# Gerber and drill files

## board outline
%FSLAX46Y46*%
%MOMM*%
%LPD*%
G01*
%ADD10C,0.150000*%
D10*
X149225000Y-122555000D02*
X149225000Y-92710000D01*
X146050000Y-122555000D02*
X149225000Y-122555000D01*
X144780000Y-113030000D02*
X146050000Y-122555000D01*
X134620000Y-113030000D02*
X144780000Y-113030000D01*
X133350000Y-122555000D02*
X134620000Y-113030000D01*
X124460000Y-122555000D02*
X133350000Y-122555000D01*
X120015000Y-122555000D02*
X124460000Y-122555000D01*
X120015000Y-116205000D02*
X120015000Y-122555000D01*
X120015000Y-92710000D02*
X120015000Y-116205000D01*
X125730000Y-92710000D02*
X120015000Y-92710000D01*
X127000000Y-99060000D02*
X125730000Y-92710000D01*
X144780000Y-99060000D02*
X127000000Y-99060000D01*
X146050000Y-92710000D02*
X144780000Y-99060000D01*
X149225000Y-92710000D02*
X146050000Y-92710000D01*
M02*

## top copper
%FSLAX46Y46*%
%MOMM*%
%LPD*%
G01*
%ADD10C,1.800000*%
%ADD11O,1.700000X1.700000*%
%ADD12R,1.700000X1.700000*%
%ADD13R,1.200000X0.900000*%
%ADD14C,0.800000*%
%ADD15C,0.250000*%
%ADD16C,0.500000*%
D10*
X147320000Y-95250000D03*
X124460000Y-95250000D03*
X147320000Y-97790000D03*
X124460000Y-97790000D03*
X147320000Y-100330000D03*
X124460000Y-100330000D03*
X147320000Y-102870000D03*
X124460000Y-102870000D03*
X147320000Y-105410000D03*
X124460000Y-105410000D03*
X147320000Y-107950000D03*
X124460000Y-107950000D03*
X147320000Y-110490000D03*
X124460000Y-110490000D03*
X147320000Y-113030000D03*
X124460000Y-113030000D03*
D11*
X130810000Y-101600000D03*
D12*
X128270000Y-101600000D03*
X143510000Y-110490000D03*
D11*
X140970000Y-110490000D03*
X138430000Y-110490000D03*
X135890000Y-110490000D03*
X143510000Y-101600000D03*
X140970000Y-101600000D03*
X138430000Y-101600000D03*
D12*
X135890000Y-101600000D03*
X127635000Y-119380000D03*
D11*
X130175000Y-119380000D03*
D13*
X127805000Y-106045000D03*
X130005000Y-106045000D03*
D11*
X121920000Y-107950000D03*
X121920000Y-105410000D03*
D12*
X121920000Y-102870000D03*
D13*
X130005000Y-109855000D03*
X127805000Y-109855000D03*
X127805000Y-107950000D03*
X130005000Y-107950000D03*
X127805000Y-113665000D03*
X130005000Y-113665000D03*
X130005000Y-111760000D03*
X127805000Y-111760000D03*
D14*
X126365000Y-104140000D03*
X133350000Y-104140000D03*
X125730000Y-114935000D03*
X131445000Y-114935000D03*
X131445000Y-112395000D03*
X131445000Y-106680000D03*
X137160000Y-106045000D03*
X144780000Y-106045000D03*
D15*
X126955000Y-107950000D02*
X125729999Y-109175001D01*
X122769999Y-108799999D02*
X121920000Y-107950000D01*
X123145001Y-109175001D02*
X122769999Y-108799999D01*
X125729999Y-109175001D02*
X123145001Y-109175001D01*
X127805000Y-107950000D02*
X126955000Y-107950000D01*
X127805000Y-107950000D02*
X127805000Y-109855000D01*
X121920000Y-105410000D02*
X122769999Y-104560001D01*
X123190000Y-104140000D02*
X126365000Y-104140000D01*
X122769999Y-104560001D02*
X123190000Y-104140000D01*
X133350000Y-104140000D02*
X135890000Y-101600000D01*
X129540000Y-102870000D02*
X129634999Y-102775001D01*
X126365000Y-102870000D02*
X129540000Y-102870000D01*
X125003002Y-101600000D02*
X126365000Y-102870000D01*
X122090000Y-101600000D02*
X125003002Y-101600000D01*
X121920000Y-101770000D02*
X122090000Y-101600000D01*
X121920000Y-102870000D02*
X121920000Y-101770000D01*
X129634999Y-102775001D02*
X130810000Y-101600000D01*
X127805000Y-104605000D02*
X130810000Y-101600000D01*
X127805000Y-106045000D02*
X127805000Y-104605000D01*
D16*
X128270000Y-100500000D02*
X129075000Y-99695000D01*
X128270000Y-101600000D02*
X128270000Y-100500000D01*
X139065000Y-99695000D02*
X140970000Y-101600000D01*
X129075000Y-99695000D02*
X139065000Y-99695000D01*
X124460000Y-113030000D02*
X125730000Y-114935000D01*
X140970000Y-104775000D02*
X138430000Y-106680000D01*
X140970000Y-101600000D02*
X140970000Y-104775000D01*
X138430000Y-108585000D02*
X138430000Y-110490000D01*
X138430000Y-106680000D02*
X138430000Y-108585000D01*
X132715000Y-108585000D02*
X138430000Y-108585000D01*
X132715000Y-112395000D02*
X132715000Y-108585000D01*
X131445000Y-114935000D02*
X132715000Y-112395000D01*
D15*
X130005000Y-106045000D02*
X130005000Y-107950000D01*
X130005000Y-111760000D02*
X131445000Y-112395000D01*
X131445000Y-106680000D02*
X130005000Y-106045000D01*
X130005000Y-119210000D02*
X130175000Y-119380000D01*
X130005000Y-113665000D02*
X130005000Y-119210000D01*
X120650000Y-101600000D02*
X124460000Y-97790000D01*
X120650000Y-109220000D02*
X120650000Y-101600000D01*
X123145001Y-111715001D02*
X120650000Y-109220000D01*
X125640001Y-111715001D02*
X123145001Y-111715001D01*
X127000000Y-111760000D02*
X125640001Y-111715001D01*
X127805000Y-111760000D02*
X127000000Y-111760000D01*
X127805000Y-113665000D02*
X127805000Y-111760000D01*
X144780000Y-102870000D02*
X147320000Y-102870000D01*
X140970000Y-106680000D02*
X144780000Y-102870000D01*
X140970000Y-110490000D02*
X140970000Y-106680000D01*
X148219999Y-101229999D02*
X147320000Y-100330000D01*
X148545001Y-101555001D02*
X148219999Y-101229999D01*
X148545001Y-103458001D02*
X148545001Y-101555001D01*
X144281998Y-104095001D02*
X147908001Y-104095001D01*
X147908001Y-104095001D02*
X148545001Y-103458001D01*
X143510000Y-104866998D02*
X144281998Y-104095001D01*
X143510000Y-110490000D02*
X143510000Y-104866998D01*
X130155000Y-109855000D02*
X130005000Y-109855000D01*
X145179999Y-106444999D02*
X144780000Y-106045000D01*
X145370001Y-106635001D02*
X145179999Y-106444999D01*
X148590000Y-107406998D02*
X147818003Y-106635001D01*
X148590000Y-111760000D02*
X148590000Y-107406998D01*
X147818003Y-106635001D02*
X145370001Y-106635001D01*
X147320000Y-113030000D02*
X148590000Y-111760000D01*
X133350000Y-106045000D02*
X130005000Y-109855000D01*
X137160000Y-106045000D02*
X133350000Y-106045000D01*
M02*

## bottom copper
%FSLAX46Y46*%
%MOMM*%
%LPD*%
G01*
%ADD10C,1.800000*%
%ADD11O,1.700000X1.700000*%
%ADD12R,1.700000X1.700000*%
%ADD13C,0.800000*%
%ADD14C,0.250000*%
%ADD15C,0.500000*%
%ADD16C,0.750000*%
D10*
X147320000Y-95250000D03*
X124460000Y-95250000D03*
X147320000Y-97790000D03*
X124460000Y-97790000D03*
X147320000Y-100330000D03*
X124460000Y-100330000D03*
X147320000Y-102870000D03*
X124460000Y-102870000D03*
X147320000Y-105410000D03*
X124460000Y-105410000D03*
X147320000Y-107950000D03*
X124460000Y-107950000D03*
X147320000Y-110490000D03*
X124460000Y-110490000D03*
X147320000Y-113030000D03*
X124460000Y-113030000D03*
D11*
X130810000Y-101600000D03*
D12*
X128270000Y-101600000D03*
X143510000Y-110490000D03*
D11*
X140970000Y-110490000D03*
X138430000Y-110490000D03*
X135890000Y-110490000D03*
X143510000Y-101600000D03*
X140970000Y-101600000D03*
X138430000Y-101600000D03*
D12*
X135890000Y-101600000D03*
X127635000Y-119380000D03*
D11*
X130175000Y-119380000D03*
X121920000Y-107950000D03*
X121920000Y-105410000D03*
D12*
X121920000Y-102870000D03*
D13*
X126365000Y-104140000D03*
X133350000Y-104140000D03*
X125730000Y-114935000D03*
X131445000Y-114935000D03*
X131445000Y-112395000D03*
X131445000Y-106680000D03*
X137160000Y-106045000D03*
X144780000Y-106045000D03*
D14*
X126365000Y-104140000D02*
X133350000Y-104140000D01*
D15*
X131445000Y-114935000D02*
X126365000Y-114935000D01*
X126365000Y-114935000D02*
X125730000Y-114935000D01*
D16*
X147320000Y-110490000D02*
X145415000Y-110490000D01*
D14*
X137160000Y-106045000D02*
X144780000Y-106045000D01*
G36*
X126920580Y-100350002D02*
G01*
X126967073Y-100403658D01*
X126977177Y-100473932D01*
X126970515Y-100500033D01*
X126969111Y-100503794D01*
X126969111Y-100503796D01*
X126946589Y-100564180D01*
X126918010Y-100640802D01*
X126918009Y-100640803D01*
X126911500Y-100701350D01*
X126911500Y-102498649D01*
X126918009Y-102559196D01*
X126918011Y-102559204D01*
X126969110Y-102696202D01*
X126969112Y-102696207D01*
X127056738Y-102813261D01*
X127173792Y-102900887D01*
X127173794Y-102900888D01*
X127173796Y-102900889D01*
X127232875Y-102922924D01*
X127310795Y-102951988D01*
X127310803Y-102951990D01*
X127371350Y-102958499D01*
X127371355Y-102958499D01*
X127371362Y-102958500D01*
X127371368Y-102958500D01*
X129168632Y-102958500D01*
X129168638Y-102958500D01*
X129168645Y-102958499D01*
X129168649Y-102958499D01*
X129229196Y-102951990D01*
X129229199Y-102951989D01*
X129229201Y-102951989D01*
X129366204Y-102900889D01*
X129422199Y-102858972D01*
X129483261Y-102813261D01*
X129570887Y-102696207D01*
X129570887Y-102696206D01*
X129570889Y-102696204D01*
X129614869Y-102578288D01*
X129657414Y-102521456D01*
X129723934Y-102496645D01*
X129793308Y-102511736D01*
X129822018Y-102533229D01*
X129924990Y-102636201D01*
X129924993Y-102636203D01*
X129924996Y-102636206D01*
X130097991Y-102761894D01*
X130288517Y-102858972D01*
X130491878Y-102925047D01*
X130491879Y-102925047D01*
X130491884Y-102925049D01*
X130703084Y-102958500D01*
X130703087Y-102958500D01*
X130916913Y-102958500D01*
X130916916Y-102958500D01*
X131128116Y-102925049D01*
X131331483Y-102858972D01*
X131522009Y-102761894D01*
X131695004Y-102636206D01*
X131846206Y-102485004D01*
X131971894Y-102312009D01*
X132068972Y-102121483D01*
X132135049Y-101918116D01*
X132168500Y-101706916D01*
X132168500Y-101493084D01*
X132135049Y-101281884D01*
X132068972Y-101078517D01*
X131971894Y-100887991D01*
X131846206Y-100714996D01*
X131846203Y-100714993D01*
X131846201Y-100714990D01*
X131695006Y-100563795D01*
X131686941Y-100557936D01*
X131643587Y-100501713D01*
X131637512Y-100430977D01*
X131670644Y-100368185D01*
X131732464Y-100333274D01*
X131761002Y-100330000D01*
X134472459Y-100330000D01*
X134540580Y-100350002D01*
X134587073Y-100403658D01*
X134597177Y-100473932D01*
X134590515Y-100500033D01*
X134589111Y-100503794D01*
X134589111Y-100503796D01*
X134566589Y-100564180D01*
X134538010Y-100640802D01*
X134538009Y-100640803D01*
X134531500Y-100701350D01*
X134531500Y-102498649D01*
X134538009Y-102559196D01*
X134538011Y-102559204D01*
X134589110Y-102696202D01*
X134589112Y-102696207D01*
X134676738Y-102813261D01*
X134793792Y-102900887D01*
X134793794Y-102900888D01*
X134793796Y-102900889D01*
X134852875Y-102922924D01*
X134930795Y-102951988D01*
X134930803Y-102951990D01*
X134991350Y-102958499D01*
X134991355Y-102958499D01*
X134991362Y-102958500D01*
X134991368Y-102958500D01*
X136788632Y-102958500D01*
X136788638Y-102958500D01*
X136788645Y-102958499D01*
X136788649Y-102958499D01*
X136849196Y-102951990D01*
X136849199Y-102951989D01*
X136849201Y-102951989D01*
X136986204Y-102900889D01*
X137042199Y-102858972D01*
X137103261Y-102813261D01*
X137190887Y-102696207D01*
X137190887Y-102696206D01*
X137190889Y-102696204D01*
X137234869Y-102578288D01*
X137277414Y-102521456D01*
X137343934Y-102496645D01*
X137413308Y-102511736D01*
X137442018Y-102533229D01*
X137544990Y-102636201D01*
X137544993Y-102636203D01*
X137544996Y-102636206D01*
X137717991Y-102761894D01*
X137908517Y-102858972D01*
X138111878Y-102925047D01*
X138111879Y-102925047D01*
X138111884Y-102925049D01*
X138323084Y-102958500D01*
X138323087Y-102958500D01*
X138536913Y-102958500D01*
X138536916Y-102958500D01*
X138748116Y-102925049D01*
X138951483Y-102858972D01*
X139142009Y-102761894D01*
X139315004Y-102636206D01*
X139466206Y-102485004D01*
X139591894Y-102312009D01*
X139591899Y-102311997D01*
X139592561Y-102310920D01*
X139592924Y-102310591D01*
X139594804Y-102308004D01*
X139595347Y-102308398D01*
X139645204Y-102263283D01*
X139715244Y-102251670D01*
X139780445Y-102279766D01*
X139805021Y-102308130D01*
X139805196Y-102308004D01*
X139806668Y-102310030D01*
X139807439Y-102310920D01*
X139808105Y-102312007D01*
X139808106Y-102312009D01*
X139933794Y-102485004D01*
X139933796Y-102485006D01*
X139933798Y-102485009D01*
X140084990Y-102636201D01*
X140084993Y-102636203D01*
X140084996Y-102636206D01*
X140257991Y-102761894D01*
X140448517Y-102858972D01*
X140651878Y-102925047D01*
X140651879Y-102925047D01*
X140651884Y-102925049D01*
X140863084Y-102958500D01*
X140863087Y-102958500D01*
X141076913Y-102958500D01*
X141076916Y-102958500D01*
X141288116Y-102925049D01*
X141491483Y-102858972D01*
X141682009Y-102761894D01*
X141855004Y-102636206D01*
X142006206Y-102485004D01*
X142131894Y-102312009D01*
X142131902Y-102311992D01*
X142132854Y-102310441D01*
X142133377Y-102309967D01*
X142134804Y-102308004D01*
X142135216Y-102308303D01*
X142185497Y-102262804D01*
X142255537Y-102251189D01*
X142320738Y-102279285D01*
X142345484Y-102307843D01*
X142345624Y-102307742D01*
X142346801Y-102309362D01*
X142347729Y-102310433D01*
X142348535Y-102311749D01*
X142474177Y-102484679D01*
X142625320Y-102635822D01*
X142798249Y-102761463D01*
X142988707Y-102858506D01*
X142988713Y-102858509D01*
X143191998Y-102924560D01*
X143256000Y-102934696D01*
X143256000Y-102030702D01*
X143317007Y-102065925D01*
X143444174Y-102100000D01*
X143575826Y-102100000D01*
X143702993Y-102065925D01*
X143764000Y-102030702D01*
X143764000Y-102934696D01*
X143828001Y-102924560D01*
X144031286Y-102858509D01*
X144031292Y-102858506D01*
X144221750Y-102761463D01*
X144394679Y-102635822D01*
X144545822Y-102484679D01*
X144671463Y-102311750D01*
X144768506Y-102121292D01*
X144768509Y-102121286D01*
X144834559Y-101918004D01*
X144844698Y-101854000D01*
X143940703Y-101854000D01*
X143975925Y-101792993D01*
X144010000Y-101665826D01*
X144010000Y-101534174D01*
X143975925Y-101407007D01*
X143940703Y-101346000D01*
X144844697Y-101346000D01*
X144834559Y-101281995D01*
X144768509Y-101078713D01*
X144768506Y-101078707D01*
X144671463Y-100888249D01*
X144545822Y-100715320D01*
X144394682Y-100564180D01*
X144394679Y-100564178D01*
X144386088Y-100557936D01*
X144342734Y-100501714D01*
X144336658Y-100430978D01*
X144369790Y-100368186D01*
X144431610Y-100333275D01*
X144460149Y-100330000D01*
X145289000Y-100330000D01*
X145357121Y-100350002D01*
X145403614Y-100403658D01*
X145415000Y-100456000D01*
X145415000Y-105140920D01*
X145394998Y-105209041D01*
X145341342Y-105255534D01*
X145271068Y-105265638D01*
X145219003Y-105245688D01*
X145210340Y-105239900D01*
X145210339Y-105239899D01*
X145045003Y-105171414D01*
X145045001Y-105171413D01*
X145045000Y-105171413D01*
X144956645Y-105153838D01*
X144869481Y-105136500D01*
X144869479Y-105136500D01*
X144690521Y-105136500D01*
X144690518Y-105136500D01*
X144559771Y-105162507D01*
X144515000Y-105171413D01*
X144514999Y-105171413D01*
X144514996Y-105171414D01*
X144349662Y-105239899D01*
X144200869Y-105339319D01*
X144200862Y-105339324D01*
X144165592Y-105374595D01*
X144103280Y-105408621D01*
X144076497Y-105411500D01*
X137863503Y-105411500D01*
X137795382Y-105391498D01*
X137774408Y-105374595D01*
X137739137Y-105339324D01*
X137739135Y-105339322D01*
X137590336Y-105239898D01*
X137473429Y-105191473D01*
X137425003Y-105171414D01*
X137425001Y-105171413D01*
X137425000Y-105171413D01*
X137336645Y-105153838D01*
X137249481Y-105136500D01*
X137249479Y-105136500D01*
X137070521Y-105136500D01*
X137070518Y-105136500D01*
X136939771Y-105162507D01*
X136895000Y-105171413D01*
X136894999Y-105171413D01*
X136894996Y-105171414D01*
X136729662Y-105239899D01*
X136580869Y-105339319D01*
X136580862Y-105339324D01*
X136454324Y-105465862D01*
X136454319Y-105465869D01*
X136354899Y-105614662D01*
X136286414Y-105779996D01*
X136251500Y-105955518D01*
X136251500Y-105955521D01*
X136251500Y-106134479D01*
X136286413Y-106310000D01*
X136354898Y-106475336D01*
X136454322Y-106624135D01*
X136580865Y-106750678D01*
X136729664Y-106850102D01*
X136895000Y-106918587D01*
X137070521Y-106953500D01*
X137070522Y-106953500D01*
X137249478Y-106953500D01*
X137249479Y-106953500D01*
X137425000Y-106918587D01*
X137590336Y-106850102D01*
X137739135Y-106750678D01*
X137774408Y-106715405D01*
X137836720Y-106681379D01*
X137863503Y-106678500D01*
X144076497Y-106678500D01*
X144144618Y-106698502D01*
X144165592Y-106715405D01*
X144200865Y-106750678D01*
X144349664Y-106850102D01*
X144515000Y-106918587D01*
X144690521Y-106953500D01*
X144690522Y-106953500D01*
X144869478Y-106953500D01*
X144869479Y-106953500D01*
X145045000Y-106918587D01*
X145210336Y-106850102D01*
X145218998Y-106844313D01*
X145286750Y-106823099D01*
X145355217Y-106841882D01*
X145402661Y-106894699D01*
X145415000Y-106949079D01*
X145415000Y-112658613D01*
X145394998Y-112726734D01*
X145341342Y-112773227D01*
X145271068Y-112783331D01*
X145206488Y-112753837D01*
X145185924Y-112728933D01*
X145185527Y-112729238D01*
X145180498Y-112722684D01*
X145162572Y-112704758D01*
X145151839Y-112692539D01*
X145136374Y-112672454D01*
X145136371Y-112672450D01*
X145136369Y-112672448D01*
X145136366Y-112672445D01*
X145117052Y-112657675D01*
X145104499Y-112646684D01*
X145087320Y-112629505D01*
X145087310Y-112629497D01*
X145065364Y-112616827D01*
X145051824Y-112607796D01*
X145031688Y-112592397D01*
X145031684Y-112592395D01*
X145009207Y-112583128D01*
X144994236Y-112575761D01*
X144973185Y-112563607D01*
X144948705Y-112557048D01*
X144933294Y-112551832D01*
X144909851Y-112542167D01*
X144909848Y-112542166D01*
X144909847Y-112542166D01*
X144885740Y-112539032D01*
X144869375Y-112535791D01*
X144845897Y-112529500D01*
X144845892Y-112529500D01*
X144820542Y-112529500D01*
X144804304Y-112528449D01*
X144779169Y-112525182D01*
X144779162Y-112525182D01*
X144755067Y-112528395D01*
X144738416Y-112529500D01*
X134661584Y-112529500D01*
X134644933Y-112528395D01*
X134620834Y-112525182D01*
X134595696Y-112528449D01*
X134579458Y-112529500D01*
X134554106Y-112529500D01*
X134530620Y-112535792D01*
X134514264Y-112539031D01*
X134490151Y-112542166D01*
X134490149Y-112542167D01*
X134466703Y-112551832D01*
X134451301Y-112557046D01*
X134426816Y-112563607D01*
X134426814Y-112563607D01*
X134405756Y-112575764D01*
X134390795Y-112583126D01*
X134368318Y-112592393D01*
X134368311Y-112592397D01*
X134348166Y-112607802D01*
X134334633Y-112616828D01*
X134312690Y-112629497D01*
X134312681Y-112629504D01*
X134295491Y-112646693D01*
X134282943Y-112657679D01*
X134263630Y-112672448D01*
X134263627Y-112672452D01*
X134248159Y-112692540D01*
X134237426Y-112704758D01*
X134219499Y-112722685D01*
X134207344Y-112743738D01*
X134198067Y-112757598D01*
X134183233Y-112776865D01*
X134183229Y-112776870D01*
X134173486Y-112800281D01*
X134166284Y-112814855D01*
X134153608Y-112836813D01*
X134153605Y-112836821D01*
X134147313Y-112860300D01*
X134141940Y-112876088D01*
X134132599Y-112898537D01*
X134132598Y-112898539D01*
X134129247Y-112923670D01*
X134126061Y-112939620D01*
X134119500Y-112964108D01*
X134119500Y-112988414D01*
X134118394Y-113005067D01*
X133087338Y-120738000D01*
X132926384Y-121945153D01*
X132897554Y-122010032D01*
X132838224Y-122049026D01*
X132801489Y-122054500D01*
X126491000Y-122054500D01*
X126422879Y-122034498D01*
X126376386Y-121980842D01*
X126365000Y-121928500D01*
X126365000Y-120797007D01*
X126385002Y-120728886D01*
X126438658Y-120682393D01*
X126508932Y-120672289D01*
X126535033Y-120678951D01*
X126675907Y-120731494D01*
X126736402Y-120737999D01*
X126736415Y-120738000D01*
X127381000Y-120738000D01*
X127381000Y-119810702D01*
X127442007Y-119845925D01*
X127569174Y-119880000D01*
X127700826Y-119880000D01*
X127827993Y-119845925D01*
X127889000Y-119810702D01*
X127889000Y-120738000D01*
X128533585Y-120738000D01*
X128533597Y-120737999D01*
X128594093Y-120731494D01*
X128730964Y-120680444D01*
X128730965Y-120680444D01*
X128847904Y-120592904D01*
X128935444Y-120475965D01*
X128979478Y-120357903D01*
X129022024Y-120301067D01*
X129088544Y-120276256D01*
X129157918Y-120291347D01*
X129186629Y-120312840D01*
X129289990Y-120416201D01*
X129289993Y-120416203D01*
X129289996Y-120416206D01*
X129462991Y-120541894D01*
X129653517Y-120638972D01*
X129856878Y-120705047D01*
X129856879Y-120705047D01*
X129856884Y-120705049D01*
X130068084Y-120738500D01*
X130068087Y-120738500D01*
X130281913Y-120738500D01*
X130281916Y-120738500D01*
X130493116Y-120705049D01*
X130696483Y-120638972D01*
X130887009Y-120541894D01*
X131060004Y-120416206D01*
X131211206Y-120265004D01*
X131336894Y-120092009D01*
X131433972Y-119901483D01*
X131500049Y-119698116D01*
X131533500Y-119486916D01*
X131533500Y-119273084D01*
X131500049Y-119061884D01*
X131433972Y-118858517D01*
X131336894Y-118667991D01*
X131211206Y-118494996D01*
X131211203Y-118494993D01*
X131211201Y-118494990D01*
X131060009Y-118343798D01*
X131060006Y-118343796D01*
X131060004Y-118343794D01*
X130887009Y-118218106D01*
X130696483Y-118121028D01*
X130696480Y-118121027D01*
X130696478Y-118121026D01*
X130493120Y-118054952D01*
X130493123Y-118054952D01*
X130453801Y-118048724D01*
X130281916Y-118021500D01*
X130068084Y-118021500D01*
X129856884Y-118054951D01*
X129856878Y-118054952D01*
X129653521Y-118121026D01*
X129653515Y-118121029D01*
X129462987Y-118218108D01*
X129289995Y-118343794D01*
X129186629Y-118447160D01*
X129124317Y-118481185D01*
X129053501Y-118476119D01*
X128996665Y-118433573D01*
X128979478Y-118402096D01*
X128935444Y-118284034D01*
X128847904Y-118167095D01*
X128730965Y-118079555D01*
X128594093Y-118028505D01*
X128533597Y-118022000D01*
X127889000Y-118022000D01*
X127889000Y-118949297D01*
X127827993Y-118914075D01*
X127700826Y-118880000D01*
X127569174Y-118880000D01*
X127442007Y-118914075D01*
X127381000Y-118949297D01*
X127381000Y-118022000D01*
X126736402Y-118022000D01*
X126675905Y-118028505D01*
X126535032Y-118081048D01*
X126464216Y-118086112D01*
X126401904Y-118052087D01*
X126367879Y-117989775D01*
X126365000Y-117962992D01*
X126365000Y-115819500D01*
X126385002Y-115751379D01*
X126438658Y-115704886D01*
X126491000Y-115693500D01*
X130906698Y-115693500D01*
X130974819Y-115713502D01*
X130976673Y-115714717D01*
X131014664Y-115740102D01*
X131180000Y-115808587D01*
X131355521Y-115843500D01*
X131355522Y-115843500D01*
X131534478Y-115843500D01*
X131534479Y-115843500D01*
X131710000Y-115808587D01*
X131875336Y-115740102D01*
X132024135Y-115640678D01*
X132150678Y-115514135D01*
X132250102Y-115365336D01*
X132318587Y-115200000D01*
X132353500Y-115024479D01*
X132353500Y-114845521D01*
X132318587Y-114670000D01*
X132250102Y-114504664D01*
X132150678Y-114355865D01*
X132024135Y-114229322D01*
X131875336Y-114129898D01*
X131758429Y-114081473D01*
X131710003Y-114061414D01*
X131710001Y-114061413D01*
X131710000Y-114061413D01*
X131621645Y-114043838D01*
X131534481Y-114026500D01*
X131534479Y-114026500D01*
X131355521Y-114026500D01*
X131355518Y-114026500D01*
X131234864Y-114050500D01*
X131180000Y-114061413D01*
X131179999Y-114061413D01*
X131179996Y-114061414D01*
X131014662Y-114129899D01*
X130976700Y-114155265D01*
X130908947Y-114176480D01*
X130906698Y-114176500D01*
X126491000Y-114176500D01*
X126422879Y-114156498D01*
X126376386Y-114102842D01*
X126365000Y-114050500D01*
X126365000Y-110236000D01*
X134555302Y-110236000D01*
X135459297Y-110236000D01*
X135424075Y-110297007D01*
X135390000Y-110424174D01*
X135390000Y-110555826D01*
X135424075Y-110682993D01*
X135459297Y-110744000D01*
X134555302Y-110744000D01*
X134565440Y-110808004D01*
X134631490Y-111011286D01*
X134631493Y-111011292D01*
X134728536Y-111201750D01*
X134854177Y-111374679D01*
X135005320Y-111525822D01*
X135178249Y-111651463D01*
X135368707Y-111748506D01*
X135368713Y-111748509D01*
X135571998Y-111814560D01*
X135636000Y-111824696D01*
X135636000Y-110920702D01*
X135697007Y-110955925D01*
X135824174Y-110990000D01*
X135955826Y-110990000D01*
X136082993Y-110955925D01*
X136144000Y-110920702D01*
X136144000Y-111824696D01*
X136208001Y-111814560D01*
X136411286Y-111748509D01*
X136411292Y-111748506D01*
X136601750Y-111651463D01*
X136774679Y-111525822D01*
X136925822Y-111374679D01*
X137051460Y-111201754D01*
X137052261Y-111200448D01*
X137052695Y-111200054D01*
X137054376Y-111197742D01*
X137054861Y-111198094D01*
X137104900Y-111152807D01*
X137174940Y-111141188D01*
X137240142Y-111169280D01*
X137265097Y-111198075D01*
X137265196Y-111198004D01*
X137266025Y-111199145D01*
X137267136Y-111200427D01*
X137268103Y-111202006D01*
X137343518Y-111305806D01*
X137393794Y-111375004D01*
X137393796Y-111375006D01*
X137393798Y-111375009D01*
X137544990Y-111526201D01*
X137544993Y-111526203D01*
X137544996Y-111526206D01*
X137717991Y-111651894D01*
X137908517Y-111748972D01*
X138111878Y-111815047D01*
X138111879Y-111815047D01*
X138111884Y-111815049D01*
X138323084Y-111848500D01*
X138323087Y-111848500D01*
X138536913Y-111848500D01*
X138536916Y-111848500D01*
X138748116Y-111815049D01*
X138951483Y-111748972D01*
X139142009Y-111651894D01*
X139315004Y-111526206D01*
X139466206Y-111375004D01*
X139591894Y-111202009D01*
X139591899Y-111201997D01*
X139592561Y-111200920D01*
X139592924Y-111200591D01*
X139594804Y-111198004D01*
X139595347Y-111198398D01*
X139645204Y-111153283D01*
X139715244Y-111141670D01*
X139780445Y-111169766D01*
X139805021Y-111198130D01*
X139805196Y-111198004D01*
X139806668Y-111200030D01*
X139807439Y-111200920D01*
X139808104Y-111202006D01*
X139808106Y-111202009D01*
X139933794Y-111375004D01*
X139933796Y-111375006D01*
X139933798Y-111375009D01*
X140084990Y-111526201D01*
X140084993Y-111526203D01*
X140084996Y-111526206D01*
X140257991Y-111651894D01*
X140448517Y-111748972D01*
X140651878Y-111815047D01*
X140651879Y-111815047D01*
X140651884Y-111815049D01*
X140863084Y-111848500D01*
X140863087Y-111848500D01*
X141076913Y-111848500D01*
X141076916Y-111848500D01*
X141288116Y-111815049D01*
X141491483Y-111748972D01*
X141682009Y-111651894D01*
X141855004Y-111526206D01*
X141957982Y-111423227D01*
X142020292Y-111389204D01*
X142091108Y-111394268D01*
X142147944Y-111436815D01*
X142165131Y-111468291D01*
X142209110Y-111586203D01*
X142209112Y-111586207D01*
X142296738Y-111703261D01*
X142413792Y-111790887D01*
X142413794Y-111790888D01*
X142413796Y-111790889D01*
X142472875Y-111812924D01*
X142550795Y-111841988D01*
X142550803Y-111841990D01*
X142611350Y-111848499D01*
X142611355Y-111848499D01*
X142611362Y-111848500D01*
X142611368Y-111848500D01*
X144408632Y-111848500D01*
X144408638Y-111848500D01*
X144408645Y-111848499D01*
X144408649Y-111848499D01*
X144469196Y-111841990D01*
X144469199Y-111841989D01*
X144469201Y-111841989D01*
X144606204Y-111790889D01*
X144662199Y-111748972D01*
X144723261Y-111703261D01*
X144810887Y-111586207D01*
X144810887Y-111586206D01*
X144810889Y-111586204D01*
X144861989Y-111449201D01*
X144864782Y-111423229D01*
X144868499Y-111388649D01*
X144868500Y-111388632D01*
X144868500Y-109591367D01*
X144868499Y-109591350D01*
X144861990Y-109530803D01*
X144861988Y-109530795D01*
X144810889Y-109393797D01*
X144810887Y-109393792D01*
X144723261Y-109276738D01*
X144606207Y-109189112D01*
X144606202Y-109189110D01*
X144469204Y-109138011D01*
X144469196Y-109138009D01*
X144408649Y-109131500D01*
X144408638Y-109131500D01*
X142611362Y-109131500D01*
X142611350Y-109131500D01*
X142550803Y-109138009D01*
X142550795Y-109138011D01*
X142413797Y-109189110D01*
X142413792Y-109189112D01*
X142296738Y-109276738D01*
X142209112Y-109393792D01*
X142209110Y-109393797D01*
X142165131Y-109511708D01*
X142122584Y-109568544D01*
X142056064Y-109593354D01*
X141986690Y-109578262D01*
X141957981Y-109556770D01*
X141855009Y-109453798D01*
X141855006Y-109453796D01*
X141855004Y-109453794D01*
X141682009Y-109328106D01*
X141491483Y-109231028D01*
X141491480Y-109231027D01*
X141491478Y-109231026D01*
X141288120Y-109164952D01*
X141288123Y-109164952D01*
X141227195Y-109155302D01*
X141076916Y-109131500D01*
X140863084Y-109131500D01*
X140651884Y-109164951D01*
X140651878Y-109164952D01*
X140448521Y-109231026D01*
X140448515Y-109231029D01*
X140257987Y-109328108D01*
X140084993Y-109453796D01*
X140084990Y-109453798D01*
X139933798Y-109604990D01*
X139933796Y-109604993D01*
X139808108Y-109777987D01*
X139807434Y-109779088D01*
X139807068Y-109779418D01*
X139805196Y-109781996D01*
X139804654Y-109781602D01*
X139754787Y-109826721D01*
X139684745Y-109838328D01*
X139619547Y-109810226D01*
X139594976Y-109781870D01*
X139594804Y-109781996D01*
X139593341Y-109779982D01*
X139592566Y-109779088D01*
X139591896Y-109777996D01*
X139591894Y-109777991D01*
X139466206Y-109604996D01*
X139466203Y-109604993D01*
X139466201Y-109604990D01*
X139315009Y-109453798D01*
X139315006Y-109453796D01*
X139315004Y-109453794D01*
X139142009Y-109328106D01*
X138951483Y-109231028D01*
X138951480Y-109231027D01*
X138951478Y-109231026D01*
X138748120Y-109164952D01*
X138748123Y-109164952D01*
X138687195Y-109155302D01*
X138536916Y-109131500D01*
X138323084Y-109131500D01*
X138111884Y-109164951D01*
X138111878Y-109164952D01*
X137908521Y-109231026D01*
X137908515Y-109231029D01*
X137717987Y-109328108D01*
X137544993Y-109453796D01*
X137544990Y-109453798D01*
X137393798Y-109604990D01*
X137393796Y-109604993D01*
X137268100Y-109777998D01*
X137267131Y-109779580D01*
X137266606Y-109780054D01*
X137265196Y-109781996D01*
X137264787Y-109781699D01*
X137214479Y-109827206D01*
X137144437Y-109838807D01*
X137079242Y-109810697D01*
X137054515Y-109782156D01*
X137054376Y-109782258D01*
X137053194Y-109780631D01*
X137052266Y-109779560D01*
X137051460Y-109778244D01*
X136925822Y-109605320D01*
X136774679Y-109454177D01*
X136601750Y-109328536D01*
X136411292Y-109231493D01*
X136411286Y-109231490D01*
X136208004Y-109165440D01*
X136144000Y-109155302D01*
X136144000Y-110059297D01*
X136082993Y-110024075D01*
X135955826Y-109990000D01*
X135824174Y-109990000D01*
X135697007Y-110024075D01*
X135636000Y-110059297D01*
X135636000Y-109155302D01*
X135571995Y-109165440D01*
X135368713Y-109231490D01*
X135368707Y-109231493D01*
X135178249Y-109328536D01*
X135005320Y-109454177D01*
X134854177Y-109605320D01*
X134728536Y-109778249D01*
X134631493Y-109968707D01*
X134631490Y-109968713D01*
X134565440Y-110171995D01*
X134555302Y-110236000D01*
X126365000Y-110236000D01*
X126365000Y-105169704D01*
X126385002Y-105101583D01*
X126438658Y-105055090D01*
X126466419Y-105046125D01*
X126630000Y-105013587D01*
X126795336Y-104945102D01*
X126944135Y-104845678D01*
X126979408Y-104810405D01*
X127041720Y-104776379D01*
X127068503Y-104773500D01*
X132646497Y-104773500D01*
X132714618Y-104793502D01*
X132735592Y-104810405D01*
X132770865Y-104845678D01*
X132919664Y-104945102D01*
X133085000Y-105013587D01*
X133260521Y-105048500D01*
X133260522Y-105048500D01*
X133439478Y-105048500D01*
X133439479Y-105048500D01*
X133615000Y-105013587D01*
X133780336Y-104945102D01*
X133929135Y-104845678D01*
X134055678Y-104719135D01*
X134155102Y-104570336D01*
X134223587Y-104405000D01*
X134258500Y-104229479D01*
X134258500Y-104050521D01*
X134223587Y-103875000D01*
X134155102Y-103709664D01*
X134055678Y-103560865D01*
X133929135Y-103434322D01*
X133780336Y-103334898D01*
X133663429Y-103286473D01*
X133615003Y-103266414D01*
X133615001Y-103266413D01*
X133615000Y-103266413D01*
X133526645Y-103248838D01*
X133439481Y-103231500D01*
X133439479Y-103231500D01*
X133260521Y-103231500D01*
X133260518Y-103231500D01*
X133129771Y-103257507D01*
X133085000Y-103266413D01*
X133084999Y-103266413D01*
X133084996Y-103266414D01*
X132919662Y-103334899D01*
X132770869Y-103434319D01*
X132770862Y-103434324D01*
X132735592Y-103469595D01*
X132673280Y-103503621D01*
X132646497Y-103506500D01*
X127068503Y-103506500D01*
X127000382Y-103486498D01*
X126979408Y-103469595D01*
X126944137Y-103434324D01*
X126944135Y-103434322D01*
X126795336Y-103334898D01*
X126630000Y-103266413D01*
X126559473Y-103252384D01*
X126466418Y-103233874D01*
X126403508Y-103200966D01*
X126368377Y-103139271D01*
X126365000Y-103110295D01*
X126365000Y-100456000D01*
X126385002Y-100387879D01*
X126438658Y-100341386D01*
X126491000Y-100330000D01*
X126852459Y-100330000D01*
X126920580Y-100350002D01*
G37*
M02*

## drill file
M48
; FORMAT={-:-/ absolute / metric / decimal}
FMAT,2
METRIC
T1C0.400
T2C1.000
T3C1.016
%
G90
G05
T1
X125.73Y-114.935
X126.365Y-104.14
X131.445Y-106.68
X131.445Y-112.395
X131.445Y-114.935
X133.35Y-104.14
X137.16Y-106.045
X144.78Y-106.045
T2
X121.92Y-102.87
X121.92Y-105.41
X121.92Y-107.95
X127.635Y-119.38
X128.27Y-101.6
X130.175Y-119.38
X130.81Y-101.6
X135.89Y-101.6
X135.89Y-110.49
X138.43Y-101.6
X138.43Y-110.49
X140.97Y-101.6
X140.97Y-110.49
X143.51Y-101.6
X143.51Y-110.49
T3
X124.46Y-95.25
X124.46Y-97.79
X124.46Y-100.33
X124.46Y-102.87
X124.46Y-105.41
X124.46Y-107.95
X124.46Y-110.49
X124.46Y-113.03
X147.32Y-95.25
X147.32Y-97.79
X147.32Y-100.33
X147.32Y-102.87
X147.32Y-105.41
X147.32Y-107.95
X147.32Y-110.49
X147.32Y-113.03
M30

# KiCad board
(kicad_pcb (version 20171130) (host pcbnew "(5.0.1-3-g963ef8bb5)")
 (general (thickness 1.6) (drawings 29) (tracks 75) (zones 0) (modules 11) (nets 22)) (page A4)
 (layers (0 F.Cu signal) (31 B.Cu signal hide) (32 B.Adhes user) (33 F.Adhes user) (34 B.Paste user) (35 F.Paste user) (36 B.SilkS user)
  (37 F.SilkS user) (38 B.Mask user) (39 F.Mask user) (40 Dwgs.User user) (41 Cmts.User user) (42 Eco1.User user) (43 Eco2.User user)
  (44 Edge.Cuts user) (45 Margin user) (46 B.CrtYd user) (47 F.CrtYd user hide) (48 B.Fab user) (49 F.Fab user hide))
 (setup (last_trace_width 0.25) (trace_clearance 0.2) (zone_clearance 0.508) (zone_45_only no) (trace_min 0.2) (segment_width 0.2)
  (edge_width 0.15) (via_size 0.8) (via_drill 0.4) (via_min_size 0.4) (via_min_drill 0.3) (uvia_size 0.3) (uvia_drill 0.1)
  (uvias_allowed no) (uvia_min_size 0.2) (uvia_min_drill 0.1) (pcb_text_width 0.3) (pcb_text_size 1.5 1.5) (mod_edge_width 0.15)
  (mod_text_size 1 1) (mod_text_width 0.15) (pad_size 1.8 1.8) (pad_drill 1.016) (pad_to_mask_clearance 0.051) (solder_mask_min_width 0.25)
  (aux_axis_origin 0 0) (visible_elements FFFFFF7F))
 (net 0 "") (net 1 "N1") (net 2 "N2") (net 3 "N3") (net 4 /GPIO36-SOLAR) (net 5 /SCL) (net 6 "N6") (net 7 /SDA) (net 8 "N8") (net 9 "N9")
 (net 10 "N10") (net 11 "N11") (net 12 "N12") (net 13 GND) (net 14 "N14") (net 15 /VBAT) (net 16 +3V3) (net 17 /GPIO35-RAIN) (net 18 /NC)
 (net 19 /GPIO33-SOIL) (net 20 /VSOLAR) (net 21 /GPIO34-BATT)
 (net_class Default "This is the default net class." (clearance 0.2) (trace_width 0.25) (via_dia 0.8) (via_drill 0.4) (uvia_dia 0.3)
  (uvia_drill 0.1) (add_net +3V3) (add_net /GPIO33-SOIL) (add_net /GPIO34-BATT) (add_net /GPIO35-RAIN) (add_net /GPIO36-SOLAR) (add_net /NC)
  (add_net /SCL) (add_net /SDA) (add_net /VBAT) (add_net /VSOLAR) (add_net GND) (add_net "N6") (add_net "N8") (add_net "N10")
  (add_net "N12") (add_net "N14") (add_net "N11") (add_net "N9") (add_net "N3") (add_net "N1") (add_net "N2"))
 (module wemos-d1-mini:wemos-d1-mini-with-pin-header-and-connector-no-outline (layer F.Cu) (at 135.89 104.14 90)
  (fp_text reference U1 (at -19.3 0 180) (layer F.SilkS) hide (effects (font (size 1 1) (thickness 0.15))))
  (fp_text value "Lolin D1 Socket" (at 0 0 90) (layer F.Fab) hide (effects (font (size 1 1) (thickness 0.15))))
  (pad 8 thru_hole circle (at 8.89 11.43 90) (size 1.8 1.8) (drill 1.016) (layers *.Cu *.Mask) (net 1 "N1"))
  (pad 9 thru_hole circle (at 8.89 -11.43 90) (size 1.8 1.8) (drill 1.016) (layers *.Cu *.Mask) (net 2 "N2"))
  (pad 7 thru_hole circle (at 6.35 11.43 90) (size 1.8 1.8) (drill 1.016) (layers *.Cu *.Mask) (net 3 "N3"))
  (pad 10 thru_hole circle (at 6.35 -11.43 90) (size 1.8 1.8) (drill 1.016) (layers *.Cu *.Mask) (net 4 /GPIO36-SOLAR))
  (pad 6 thru_hole circle (at 3.81 11.43 90) (size 1.8 1.8) (drill 1.016) (layers *.Cu *.Mask) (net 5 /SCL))
  (pad 11 thru_hole circle (at 3.81 -11.43 90) (size 1.8 1.8) (drill 1.016) (layers *.Cu *.Mask) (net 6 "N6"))
  (pad 5 thru_hole circle (at 1.27 11.43 90) (size 1.8 1.8) (drill 1.016) (layers *.Cu *.Mask) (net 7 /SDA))
  (pad 12 thru_hole circle (at 1.27 -11.43 90) (size 1.8 1.8) (drill 1.016) (layers *.Cu *.Mask) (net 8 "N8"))
  (pad 4 thru_hole circle (at -1.27 11.43 90) (size 1.8 1.8) (drill 1.016) (layers *.Cu *.Mask) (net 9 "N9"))
  (pad 13 thru_hole circle (at -1.27 -11.43 90) (size 1.8 1.8) (drill 1.016) (layers *.Cu *.Mask) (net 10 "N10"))
  (pad 3 thru_hole circle (at -3.81 11.43 90) (size 1.8 1.8) (drill 1.016) (layers *.Cu *.Mask) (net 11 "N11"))
  (pad 14 thru_hole circle (at -3.81 -11.43 90) (size 1.8 1.8) (drill 1.016) (layers *.Cu *.Mask) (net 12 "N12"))
  (pad 2 thru_hole circle (at -6.35 11.43 90) (size 1.8 1.8) (drill 1.016) (layers *.Cu *.Mask) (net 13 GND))
  (pad 15 thru_hole circle (at -6.35 -11.43 90) (size 1.8 1.8) (drill 1.016) (layers *.Cu *.Mask) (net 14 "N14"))
  (pad 1 thru_hole circle (at -8.89 11.43 90) (size 1.8 1.8) (drill 1.016) (layers *.Cu *.Mask) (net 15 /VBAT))
  (pad 16 thru_hole circle (at -8.89 -11.43 90) (size 1.8 1.8) (drill 1.016) (layers *.Cu *.Mask) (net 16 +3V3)))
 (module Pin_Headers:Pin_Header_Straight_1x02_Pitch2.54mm (layer F.Cu) (at 128.27 101.6 90)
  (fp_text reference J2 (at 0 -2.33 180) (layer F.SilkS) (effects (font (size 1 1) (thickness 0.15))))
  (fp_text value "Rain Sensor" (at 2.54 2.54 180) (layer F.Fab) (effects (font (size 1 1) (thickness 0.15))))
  (pad 2 thru_hole oval (at 0 2.54 90) (size 1.7 1.7) (drill 1) (layers *.Cu *.Mask) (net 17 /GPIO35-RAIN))
  (pad 1 thru_hole rect (at 0 0 90) (size 1.7 1.7) (drill 1) (layers *.Cu *.Mask) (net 16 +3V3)))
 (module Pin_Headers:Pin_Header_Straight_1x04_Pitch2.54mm (layer F.Cu) (at 143.51 110.49 270)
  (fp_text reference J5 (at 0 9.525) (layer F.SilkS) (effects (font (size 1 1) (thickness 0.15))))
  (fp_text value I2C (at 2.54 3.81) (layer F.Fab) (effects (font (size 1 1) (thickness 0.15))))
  (pad 1 thru_hole rect (at 0 0 270) (size 1.7 1.7) (drill 1) (layers *.Cu *.Mask) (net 5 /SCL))
  (pad 2 thru_hole oval (at 0 2.54 270) (size 1.7 1.7) (drill 1) (layers *.Cu *.Mask) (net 7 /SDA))
  (pad 3 thru_hole oval (at 0 5.08 270) (size 1.7 1.7) (drill 1) (layers *.Cu *.Mask) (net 16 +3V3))
  (pad 4 thru_hole oval (at 0 7.62 270) (size 1.7 1.7) (drill 1) (layers *.Cu *.Mask) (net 13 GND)))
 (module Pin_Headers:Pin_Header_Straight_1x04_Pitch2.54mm (layer F.Cu) (at 135.89 101.6 90)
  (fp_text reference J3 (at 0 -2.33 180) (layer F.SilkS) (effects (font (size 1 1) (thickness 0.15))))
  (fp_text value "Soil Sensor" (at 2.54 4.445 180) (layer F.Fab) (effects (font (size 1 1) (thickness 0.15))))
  (pad 4 thru_hole oval (at 0 7.62 90) (size 1.7 1.7) (drill 1) (layers *.Cu *.Mask) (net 13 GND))
  (pad 3 thru_hole oval (at 0 5.08 90) (size 1.7 1.7) (drill 1) (layers *.Cu *.Mask) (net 16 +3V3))
  (pad 2 thru_hole oval (at 0 2.54 90) (size 1.7 1.7) (drill 1) (layers *.Cu *.Mask) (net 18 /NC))
  (pad 1 thru_hole rect (at 0 0 90) (size 1.7 1.7) (drill 1) (layers *.Cu *.Mask) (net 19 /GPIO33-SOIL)))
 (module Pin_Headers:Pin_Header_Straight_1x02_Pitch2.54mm (layer F.Cu) (at 127.635 119.38 90)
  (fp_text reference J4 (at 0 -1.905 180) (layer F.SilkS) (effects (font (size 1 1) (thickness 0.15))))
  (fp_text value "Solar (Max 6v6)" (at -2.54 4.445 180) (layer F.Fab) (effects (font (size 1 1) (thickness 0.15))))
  (pad 1 thru_hole rect (at 0 0 90) (size 1.7 1.7) (drill 1) (layers *.Cu *.Mask) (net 13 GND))
  (pad 2 thru_hole oval (at 0 2.54 90) (size 1.7 1.7) (drill 1) (layers *.Cu *.Mask) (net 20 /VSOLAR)))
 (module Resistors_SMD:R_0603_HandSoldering (layer F.Cu) (at 128.905 106.045 180)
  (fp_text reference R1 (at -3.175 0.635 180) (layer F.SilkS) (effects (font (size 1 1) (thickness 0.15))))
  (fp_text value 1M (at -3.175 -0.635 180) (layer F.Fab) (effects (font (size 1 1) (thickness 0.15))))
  (pad 2 smd rect (at 1.1 0 180) (size 1.2 0.9) (layers F.Cu F.Paste F.Mask) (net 17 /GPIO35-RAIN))
  (pad 1 smd rect (at -1.1 0 180) (size 1.2 0.9) (layers F.Cu F.Paste F.Mask) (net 13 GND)))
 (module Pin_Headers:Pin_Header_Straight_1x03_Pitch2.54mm (layer F.Cu) (at 121.92 102.87)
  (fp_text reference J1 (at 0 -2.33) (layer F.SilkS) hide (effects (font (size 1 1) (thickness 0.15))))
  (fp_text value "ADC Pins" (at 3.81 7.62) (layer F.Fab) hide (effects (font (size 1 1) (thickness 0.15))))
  (pad 3 thru_hole oval (at 0 5.08) (size 1.7 1.7) (drill 1) (layers *.Cu *.Mask) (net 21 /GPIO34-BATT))
  (pad 2 thru_hole oval (at 0 2.54) (size 1.7 1.7) (drill 1) (layers *.Cu *.Mask) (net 19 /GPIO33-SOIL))
  (pad 1 thru_hole rect (at 0 0) (size 1.7 1.7) (drill 1) (layers *.Cu *.Mask) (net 17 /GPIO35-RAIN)))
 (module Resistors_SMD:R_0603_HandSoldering (layer F.Cu) (at 128.905 109.855 180)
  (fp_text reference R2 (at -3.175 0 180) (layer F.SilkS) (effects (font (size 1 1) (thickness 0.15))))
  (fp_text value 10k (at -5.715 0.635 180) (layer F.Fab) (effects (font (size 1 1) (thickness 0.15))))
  (pad 1 smd rect (at -1.1 0 180) (size 1.2 0.9) (layers F.Cu F.Paste F.Mask) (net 15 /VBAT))
  (pad 2 smd rect (at 1.1 0 180) (size 1.2 0.9) (layers F.Cu F.Paste F.Mask) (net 21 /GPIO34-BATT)))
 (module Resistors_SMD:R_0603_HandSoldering (layer F.Cu) (at 128.905 107.95)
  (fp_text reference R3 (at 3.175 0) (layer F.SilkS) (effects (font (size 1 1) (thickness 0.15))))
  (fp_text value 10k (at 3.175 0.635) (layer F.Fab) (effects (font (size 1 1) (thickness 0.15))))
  (pad 1 smd rect (at -1.1 0) (size 1.2 0.9) (layers F.Cu F.Paste F.Mask) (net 21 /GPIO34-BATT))
  (pad 2 smd rect (at 1.1 0) (size 1.2 0.9) (layers F.Cu F.Paste F.Mask) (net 13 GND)))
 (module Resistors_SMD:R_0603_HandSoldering (layer F.Cu) (at 128.905 113.665 180)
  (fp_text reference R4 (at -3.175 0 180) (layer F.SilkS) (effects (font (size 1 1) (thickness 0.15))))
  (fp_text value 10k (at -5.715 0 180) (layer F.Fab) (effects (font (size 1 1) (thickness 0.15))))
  (pad 2 smd rect (at 1.1 0 180) (size 1.2 0.9) (layers F.Cu F.Paste F.Mask) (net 4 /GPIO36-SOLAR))
  (pad 1 smd rect (at -1.1 0 180) (size 1.2 0.9) (layers F.Cu F.Paste F.Mask) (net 20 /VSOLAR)))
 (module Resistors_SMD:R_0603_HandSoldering (layer F.Cu) (at 128.905 111.76)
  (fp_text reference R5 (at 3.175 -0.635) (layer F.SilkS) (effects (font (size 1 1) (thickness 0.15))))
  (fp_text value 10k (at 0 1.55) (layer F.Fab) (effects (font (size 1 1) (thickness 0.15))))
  (pad 2 smd rect (at 1.1 0) (size 1.2 0.9) (layers F.Cu F.Paste F.Mask) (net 13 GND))
  (pad 1 smd rect (at -1.1 0) (size 1.2 0.9) (layers F.Cu F.Paste F.Mask) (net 4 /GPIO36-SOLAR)))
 (gr_line (start 149.225 122.555) (end 149.225 92.71) (layer Edge.Cuts) (width 0.15))
 (gr_line (start 146.05 122.555) (end 149.225 122.555) (layer Edge.Cuts) (width 0.15))
 (gr_line (start 144.78 113.03) (end 146.05 122.555) (layer Edge.Cuts) (width 0.15))
 (gr_line (start 134.62 113.03) (end 144.78 113.03) (layer Edge.Cuts) (width 0.15))
 (gr_line (start 133.35 122.555) (end 134.62 113.03) (layer Edge.Cuts) (width 0.15))
 (gr_line (start 124.46 122.555) (end 133.35 122.555) (layer Edge.Cuts) (width 0.15))
 (gr_line (start 120.015 122.555) (end 124.46 122.555) (layer Edge.Cuts) (width 0.15))
 (gr_line (start 120.015 116.205) (end 120.015 122.555) (layer Edge.Cuts) (width 0.15))
 (gr_line (start 120.015 92.71) (end 120.015 116.205) (layer Edge.Cuts) (width 0.15))
 (gr_line (start 125.73 92.71) (end 120.015 92.71) (layer Edge.Cuts) (width 0.15))
 (gr_line (start 127 99.06) (end 125.73 92.71) (layer Edge.Cuts) (width 0.15))
 (gr_line (start 144.78 99.06) (end 127 99.06) (layer Edge.Cuts) (width 0.15))
 (gr_line (start 146.05 92.71) (end 144.78 99.06) (layer Edge.Cuts) (width 0.15))
 (gr_line (start 149.225 92.71) (end 146.05 92.71) (layer Edge.Cuts) (width 0.15))
 (segment (start 126.955 107.95) (end 125.729999 109.175001) (width 0.25) (layer F.Cu) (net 21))
 (segment (start 122.769999 108.799999) (end 121.92 107.95) (width 0.25) (layer F.Cu) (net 21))
 (segment (start 123.145001 109.175001) (end 122.769999 108.799999) (width 0.25) (layer F.Cu) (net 21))
 (segment (start 125.729999 109.175001) (end 123.145001 109.175001) (width 0.25) (layer F.Cu) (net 21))
 (segment (start 127.805 107.95) (end 126.955 107.95) (width 0.25) (layer F.Cu) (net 21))
 (segment (start 127.805 107.95) (end 127.805 109.855) (width 0.25) (layer F.Cu) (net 21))
 (segment (start 121.92 105.41) (end 122.769999 104.560001) (width 0.25) (layer F.Cu) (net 19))
 (via (at 126.365 104.14) (size 0.8) (drill 0.4) (layers F.Cu B.Cu) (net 19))
 (segment (start 123.19 104.14) (end 126.365 104.14) (width 0.25) (layer F.Cu) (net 19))
 (segment (start 122.769999 104.560001) (end 123.19 104.14) (width 0.25) (layer F.Cu) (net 19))
 (segment (start 133.35 104.14) (end 135.89 101.6) (width 0.25) (layer F.Cu) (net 19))
 (segment (start 126.365 104.14) (end 133.35 104.14) (width 0.25) (layer B.Cu) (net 19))
 (via (at 133.35 104.14) (size 0.8) (drill 0.4) (layers F.Cu B.Cu) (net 19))
 (segment (start 129.54 102.87) (end 129.634999 102.775001) (width 0.25) (layer F.Cu) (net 17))
 (segment (start 126.365 102.87) (end 129.54 102.87) (width 0.25) (layer F.Cu) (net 17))
 (segment (start 125.003002 101.6) (end 126.365 102.87) (width 0.25) (layer F.Cu) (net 17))
 (segment (start 122.09 101.6) (end 125.003002 101.6) (width 0.25) (layer F.Cu) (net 17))
 (segment (start 121.92 101.77) (end 122.09 101.6) (width 0.25) (layer F.Cu) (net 17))
 (segment (start 121.92 102.87) (end 121.92 101.77) (width 0.25) (layer F.Cu) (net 17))
 (segment (start 129.634999 102.775001) (end 130.81 101.6) (width 0.25) (layer F.Cu) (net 17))
 (segment (start 127.805 104.605) (end 130.81 101.6) (width 0.25) (layer F.Cu) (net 17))
 (segment (start 127.805 106.045) (end 127.805 104.605) (width 0.25) (layer F.Cu) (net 17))
 (segment (start 128.27 100.5) (end 129.075 99.695) (width 0.5) (layer F.Cu) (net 16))
 (segment (start 128.27 101.6) (end 128.27 100.5) (width 0.5) (layer F.Cu) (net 16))
 (segment (start 139.065 99.695) (end 140.97 101.6) (width 0.5) (layer F.Cu) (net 16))
 (segment (start 129.075 99.695) (end 139.065 99.695) (width 0.5) (layer F.Cu) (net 16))
 (segment (start 124.46 113.03) (end 125.73 114.935) (width 0.5) (layer F.Cu) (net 16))
 (via (at 125.73 114.935) (size 0.8) (drill 0.4) (layers F.Cu B.Cu) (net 16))
 (segment (start 140.97 104.775) (end 138.43 106.68) (width 0.5) (layer F.Cu) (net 16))
 (segment (start 140.97 101.6) (end 140.97 104.775) (width 0.5) (layer F.Cu) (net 16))
 (segment (start 138.43 108.585) (end 138.43 110.49) (width 0.5) (layer F.Cu) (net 16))
 (segment (start 138.43 106.68) (end 138.43 108.585) (width 0.5) (layer F.Cu) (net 16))
 (segment (start 131.445 114.935) (end 126.365 114.935) (width 0.5) (layer B.Cu) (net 16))
 (segment (start 126.365 114.935) (end 125.73 114.935) (width 0.5) (layer B.Cu) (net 16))
 (via (at 131.445 114.935) (size 0.8) (drill 0.4) (layers F.Cu B.Cu) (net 16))
 (segment (start 132.715 108.585) (end 138.43 108.585) (width 0.5) (layer F.Cu) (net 16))
 (segment (start 132.715 112.395) (end 132.715 108.585) (width 0.5) (layer F.Cu) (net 16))
 (segment (start 131.445 114.935) (end 132.715 112.395) (width 0.5) (layer F.Cu) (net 16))
 (segment (start 147.32 110.49) (end 145.415 110.49) (width 0.75) (layer B.Cu) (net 13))
 (segment (start 130.005 106.045) (end 130.005 107.95) (width 0.25) (layer F.Cu) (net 13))
 (segment (start 130.005 111.76) (end 131.445 112.395) (width 0.25) (layer F.Cu) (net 13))
 (via (at 131.445 112.395) (size 0.8) (drill 0.4) (layers F.Cu B.Cu) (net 13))
 (segment (start 131.445 106.68) (end 130.005 106.045) (width 0.25) (layer F.Cu) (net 13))
 (via (at 131.445 106.68) (size 0.8) (drill 0.4) (layers F.Cu B.Cu) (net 13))
 (segment (start 130.005 119.21) (end 130.175 119.38) (width 0.25) (layer F.Cu) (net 20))
 (segment (start 130.005 113.665) (end 130.005 119.21) (width 0.25) (layer F.Cu) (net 20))
 (segment (start 120.65 101.6) (end 124.46 97.79) (width 0.25) (layer F.Cu) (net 4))
 (segment (start 120.65 109.22) (end 120.65 101.6) (width 0.25) (layer F.Cu) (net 4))
 (segment (start 123.145001 111.715001) (end 120.65 109.22) (width 0.25) (layer F.Cu) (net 4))
 (segment (start 125.640001 111.715001) (end 123.145001 111.715001) (width 0.25) (layer F.Cu) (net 4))
 (segment (start 127 111.76) (end 125.640001 111.715001) (width 0.25) (layer F.Cu) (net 4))
 (segment (start 127.805 111.76) (end 127 111.76) (width 0.25) (layer F.Cu) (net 4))
 (segment (start 127.805 113.665) (end 127.805 111.76) (width 0.25) (layer F.Cu) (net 4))
 (segment (start 144.78 102.87) (end 147.32 102.87) (width 0.25) (layer F.Cu) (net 7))
 (segment (start 140.97 106.68) (end 144.78 102.87) (width 0.25) (layer F.Cu) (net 7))
 (segment (start 140.97 110.49) (end 140.97 106.68) (width 0.25) (layer F.Cu) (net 7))
 (segment (start 148.219999 101.229999) (end 147.32 100.33) (width 0.25) (layer F.Cu) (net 5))
 (segment (start 148.545001 101.555001) (end 148.219999 101.229999) (width 0.25) (layer F.Cu) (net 5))
 (segment (start 148.545001 103.458001) (end 148.545001 101.555001) (width 0.25) (layer F.Cu) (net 5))
 (segment (start 144.281998 104.095001) (end 147.908001 104.095001) (width 0.25) (layer F.Cu) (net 5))
 (segment (start 147.908001 104.095001) (end 148.545001 103.458001) (width 0.25) (layer F.Cu) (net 5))
 (segment (start 143.51 104.866998) (end 144.281998 104.095001) (width 0.25) (layer F.Cu) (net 5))
 (segment (start 143.51 110.49) (end 143.51 104.866998) (width 0.25) (layer F.Cu) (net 5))
 (via (at 137.16 106.045) (size 0.8) (drill 0.4) (layers F.Cu B.Cu) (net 15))
 (segment (start 137.16 106.045) (end 144.78 106.045) (width 0.25) (layer B.Cu) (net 15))
 (via (at 144.78 106.045) (size 0.8) (drill 0.4) (layers F.Cu B.Cu) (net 15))
 (segment (start 130.155 109.855) (end 130.005 109.855) (width 0.25) (layer F.Cu) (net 15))
 (segment (start 145.179999 106.444999) (end 144.78 106.045) (width 0.25) (layer F.Cu) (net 15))
 (segment (start 145.370001 106.635001) (end 145.179999 106.444999) (width 0.25) (layer F.Cu) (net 15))
 (segment (start 148.59 107.406998) (end 147.818003 106.635001) (width 0.25) (layer F.Cu) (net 15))
 (segment (start 148.59 111.76) (end 148.59 107.406998) (width 0.25) (layer F.Cu) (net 15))
 (segment (start 147.818003 106.635001) (end 145.370001 106.635001) (width 0.25) (layer F.Cu) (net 15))
 (segment (start 147.32 113.03) (end 148.59 111.76) (width 0.25) (layer F.Cu) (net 15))
 (segment (start 133.35 106.045) (end 130.005 109.855) (width 0.25) (layer F.Cu) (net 15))
 (segment (start 137.16 106.045) (end 133.35 106.045) (width 0.25) (layer F.Cu) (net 15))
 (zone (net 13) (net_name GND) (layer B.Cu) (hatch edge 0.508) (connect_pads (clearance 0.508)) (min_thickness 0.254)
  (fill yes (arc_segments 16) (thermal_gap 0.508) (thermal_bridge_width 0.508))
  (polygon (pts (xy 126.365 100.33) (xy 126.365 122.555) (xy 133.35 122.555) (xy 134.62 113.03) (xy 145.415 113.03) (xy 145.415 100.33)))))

